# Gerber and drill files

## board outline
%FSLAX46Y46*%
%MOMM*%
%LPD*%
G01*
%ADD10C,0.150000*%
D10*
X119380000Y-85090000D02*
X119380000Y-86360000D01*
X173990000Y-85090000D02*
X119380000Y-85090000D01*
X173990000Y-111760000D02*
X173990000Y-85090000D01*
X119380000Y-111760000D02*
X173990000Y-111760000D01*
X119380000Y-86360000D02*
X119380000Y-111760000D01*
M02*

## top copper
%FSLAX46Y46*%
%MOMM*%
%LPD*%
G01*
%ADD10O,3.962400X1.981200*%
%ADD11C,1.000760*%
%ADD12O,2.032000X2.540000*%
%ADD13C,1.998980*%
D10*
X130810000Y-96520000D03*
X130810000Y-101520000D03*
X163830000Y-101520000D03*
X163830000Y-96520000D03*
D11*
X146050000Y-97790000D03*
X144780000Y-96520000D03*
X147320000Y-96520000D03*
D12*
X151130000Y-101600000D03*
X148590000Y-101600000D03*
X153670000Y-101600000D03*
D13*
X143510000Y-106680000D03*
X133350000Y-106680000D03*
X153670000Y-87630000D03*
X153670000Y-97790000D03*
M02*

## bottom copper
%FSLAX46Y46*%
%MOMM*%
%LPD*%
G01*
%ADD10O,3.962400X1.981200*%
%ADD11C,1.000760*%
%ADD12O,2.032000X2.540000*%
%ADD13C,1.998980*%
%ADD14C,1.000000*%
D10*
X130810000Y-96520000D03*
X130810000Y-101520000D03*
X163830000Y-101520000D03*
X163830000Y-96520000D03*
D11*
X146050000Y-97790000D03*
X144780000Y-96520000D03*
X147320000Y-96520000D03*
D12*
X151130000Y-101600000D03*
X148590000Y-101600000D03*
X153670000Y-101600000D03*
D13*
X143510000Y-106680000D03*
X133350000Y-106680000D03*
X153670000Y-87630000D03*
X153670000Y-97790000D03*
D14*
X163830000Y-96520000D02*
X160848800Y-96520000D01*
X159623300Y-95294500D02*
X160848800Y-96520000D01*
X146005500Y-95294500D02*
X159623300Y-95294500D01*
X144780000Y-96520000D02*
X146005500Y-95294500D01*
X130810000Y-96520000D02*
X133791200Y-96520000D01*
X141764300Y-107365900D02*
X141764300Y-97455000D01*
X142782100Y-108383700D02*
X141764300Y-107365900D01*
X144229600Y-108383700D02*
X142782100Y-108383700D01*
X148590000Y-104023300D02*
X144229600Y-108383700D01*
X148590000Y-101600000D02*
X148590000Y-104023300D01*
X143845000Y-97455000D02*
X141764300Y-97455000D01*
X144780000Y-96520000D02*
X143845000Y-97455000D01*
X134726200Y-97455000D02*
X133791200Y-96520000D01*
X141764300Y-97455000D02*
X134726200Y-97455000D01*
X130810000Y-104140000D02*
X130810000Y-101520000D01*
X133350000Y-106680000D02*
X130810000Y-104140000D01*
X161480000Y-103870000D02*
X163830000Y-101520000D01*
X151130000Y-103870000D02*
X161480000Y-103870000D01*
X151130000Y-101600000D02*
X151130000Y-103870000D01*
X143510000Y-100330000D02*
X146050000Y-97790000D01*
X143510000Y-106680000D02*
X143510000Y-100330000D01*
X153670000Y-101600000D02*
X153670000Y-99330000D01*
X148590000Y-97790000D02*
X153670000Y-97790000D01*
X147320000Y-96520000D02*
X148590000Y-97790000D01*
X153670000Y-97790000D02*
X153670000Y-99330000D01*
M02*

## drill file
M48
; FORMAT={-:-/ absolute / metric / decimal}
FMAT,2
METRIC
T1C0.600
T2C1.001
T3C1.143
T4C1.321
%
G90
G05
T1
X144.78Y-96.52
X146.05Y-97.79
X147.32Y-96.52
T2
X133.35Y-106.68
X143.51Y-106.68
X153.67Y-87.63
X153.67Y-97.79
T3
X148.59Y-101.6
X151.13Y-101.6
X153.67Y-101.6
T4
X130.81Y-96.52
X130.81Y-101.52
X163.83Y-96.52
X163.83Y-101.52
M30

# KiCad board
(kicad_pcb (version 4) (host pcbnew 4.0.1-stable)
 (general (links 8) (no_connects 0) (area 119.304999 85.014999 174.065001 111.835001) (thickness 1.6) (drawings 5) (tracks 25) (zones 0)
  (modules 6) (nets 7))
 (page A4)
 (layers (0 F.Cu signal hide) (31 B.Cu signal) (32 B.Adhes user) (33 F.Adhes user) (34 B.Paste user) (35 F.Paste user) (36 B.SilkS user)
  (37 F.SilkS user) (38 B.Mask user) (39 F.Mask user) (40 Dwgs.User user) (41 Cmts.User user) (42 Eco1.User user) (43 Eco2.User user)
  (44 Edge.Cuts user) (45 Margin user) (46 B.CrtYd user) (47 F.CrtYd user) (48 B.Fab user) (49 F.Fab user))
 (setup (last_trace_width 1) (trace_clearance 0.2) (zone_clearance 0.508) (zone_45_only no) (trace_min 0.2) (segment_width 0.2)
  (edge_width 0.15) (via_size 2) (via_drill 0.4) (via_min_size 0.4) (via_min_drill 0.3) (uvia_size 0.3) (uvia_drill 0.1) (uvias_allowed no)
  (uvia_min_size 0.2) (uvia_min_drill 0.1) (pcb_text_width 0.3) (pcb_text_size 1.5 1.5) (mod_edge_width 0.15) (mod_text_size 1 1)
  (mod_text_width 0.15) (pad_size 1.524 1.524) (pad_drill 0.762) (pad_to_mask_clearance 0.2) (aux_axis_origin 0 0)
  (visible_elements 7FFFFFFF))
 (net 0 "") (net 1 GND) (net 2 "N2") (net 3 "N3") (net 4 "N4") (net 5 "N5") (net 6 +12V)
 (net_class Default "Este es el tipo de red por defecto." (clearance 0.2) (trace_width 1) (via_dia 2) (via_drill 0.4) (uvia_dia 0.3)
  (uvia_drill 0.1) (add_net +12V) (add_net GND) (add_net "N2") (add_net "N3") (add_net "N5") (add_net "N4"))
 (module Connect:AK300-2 (layer F.Cu) (at 130.81 96.52 270)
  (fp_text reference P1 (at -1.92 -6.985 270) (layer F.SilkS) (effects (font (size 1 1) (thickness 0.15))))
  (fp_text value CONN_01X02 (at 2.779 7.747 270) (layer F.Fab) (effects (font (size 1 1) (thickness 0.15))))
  (pad 1 thru_hole oval (at 0 0 270) (size 1.9812 3.9624) (drill 1.3208) (layers *.Cu F.Paste F.SilkS F.Mask) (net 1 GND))
  (pad 2 thru_hole oval (at 5 0 270) (size 1.9812 3.9624) (drill 1.3208) (layers *.Cu F.Paste F.SilkS F.Mask) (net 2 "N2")))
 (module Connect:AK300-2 (layer F.Cu) (at 163.83 101.52 90)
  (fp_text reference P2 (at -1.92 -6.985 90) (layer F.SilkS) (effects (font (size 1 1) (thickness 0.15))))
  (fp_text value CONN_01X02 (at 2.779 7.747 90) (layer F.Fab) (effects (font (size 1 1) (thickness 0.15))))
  (pad 1 thru_hole oval (at 0 0 90) (size 1.9812 3.9624) (drill 1.3208) (layers *.Cu F.Paste F.SilkS F.Mask) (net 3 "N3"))
  (pad 2 thru_hole oval (at 5 0 90) (size 1.9812 3.9624) (drill 1.3208) (layers *.Cu F.Paste F.SilkS F.Mask) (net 1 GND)))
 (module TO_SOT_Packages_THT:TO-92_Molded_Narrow (layer F.Cu) (at 147.32 96.52 180)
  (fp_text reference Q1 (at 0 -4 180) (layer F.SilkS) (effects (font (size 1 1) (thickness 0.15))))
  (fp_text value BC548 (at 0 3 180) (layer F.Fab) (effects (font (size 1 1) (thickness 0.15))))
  (pad 2 thru_hole circle (at 1.27 -1.27 270) (size 1.00076 1.00076) (drill 0.6) (layers *.Cu *.Mask F.SilkS) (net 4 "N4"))
  (pad 3 thru_hole circle (at 2.54 0 270) (size 1.00076 1.00076) (drill 0.6) (layers *.Cu *.Mask F.SilkS) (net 1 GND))
  (pad 1 thru_hole circle (at 0 0 270) (size 1.00076 1.00076) (drill 0.6) (layers *.Cu *.Mask F.SilkS) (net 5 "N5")))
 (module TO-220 (layer F.Cu) (at 151.13 101.6 180)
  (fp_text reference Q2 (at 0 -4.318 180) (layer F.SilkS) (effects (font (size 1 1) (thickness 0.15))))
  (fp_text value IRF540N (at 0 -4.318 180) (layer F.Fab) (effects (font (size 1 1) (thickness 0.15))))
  (pad 2 thru_hole oval (at 0 0 180) (size 2.032 2.54) (drill 1.143) (layers *.Cu *.Mask F.SilkS) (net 3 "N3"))
  (pad 3 thru_hole oval (at 2.54 0 180) (size 2.032 2.54) (drill 1.143) (layers *.Cu *.Mask F.SilkS) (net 1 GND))
  (pad 1 thru_hole oval (at -2.54 0 180) (size 2.032 2.54) (drill 1.143) (layers *.Cu *.Mask F.SilkS) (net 5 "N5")))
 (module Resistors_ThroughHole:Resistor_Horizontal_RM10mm (layer F.Cu) (at 138.43 106.68 180)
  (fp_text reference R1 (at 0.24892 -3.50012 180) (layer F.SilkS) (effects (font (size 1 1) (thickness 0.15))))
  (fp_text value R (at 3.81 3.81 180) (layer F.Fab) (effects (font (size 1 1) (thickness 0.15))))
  (pad 1 thru_hole circle (at -5.08 0 180) (size 1.99898 1.99898) (drill 1.00076) (layers *.Cu *.SilkS *.Mask) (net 4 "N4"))
  (pad 2 thru_hole circle (at 5.08 0 180) (size 1.99898 1.99898) (drill 1.00076) (layers *.Cu *.SilkS *.Mask) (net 2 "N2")))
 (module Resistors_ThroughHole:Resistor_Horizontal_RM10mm (layer F.Cu) (at 153.67 92.71 270)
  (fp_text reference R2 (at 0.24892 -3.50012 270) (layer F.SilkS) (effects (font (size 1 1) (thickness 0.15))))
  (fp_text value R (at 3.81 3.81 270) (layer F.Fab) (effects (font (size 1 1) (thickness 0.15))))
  (pad 1 thru_hole circle (at -5.08 0 270) (size 1.99898 1.99898) (drill 1.00076) (layers *.Cu *.SilkS *.Mask) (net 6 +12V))
  (pad 2 thru_hole circle (at 5.08 0 270) (size 1.99898 1.99898) (drill 1.00076) (layers *.Cu *.SilkS *.Mask) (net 5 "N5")))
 (gr_line (start 119.38 85.09) (end 119.38 86.36) (layer Edge.Cuts) (width 0.15))
 (gr_line (start 173.99 85.09) (end 119.38 85.09) (layer Edge.Cuts) (width 0.15))
 (gr_line (start 173.99 111.76) (end 173.99 85.09) (layer Edge.Cuts) (width 0.15))
 (gr_line (start 119.38 111.76) (end 173.99 111.76) (layer Edge.Cuts) (width 0.15))
 (gr_line (start 119.38 86.36) (end 119.38 111.76) (layer Edge.Cuts) (width 0.15))
 (segment (start 163.83 96.52) (end 160.8488 96.52) (width 1) (layer B.Cu) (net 1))
 (segment (start 159.6233 95.2945) (end 160.8488 96.52) (width 1) (layer B.Cu) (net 1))
 (segment (start 146.0055 95.2945) (end 159.6233 95.2945) (width 1) (layer B.Cu) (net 1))
 (segment (start 144.78 96.52) (end 146.0055 95.2945) (width 1) (layer B.Cu) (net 1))
 (segment (start 130.81 96.52) (end 133.7912 96.52) (width 1) (layer B.Cu) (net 1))
 (segment (start 141.7643 107.3659) (end 141.7643 97.455) (width 1) (layer B.Cu) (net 1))
 (segment (start 142.7821 108.3837) (end 141.7643 107.3659) (width 1) (layer B.Cu) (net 1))
 (segment (start 144.2296 108.3837) (end 142.7821 108.3837) (width 1) (layer B.Cu) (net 1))
 (segment (start 148.59 104.0233) (end 144.2296 108.3837) (width 1) (layer B.Cu) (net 1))
 (segment (start 148.59 101.6) (end 148.59 104.0233) (width 1) (layer B.Cu) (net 1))
 (segment (start 143.845 97.455) (end 141.7643 97.455) (width 1) (layer B.Cu) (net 1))
 (segment (start 144.78 96.52) (end 143.845 97.455) (width 1) (layer B.Cu) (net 1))
 (segment (start 134.7262 97.455) (end 133.7912 96.52) (width 1) (layer B.Cu) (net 1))
 (segment (start 141.7643 97.455) (end 134.7262 97.455) (width 1) (layer B.Cu) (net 1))
 (segment (start 130.81 104.14) (end 130.81 101.52) (width 1) (layer B.Cu) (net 2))
 (segment (start 133.35 106.68) (end 130.81 104.14) (width 1) (layer B.Cu) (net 2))
 (segment (start 161.48 103.87) (end 163.83 101.52) (width 1) (layer B.Cu) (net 3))
 (segment (start 151.13 103.87) (end 161.48 103.87) (width 1) (layer B.Cu) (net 3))
 (segment (start 151.13 101.6) (end 151.13 103.87) (width 1) (layer B.Cu) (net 3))
 (segment (start 143.51 100.33) (end 146.05 97.79) (width 1) (layer B.Cu) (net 4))
 (segment (start 143.51 106.68) (end 143.51 100.33) (width 1) (layer B.Cu) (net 4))
 (segment (start 153.67 101.6) (end 153.67 99.33) (width 1) (layer B.Cu) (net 5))
 (segment (start 148.59 97.79) (end 153.67 97.79) (width 1) (layer B.Cu) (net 5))
 (segment (start 147.32 96.52) (end 148.59 97.79) (width 1) (layer B.Cu) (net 5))
 (segment (start 153.67 97.79) (end 153.67 99.33) (width 1) (layer B.Cu) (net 5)))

